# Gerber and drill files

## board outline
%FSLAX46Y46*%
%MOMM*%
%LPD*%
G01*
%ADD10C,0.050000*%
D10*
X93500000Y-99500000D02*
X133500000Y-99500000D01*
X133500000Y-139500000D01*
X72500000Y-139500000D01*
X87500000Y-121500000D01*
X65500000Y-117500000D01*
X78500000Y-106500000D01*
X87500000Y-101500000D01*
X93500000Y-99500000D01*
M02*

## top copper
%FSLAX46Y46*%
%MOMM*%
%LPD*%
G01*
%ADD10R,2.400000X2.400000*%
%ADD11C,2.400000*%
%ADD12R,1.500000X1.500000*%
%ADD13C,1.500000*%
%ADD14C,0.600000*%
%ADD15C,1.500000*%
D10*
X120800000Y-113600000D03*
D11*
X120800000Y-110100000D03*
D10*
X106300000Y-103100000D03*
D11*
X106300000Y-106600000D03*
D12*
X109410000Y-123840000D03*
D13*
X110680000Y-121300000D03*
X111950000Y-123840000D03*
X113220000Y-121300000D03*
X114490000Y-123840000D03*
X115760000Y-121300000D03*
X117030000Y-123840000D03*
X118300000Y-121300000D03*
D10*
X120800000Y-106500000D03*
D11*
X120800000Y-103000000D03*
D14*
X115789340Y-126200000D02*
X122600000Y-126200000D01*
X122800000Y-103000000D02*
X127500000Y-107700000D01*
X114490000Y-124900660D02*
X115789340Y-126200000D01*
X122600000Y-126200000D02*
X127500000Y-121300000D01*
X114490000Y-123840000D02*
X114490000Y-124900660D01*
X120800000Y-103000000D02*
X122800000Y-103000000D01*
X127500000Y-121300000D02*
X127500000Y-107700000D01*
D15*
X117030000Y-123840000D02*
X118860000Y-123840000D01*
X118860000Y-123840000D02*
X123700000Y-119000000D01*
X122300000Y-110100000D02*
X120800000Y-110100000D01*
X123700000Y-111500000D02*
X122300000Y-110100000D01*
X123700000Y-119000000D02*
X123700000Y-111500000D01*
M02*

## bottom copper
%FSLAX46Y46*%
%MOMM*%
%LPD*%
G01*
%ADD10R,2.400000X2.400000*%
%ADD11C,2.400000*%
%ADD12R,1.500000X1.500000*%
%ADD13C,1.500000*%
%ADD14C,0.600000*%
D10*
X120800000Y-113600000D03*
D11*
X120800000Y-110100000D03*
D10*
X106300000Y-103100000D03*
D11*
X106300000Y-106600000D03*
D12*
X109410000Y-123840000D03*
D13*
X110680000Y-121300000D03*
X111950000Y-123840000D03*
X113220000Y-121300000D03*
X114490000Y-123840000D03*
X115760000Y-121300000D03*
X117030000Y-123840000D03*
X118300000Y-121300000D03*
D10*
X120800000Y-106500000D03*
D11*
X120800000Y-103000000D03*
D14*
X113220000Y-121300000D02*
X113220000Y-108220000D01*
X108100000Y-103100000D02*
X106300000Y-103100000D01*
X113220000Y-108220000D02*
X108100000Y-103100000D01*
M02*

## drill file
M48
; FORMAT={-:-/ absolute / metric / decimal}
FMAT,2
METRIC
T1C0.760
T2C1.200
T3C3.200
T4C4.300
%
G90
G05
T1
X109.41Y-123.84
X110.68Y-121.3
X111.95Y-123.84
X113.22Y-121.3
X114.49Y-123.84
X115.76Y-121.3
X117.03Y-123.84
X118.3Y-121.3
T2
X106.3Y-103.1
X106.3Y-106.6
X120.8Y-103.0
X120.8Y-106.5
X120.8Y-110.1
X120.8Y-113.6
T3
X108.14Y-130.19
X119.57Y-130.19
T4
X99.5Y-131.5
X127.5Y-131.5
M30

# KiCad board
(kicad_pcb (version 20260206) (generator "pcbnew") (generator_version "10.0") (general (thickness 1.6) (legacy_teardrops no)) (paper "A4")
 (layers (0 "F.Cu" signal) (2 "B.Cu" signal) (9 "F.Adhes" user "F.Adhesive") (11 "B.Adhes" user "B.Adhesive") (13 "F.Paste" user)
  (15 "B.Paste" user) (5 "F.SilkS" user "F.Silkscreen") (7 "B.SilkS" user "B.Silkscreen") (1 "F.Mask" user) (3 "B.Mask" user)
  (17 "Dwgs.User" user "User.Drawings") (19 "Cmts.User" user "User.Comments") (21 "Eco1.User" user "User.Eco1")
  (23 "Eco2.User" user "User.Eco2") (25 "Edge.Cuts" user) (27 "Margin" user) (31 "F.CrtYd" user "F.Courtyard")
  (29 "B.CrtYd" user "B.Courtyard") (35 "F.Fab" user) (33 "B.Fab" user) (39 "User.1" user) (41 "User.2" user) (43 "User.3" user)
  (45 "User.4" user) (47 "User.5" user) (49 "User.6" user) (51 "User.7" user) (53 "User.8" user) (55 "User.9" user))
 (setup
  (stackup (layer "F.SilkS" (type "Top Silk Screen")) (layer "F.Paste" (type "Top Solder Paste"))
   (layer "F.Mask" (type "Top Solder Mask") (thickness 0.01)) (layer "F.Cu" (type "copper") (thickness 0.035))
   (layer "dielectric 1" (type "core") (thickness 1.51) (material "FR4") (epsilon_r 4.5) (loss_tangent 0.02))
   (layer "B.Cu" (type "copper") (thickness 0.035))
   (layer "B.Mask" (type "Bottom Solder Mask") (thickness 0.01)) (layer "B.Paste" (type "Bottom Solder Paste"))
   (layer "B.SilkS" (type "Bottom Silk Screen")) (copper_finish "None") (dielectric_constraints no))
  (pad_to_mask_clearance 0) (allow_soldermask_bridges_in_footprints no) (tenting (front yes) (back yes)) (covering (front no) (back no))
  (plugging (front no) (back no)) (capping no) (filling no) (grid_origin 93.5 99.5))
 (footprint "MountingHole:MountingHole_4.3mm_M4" (layer "F.Cu") (at 127.5 131.5)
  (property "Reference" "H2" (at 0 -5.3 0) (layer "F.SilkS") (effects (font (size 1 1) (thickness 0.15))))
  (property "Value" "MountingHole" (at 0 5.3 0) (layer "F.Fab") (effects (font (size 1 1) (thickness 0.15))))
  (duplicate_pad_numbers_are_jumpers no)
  (pad "" np_thru_hole circle (at 0 0) (size 4.3 4.3) (drill 4.3) (layers "*.Cu" "*.Mask")))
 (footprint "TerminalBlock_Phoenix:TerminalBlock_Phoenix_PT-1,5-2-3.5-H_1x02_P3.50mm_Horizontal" (layer "F.Cu") (at 120.8 113.6 90)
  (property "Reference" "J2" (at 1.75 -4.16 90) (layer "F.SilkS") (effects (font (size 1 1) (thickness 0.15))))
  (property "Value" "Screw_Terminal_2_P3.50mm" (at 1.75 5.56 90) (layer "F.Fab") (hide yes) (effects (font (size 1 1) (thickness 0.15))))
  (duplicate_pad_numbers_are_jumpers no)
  (pad "1" thru_hole rect (at 0 0 90) (size 2.4 2.4) (drill 1.2) (layers "*.Cu" "*.Mask") (remove_unused_layers no) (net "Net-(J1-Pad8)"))
  (pad "2" thru_hole circle (at 3.5 0 90) (size 2.4 2.4) (drill 1.2) (layers "*.Cu" "*.Mask") (remove_unused_layers no)
   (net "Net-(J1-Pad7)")))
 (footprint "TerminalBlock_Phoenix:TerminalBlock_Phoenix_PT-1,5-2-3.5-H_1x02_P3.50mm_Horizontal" (layer "F.Cu") (at 106.3 103.1 -90)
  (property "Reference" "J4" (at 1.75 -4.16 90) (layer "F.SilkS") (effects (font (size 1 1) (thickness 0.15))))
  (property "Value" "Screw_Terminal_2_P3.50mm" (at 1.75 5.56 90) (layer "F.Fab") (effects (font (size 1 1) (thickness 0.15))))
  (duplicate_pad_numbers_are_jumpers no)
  (pad "1" thru_hole rect (at 0 0 270) (size 2.4 2.4) (drill 1.2) (layers "*.Cu" "*.Mask") (remove_unused_layers no) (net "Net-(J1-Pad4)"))
  (pad "2" thru_hole circle (at 3.5 0 270) (size 2.4 2.4) (drill 1.2) (layers "*.Cu" "*.Mask") (remove_unused_layers no)
   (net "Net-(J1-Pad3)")))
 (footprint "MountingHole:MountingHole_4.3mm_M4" (layer "F.Cu") (at 99.5 131.5)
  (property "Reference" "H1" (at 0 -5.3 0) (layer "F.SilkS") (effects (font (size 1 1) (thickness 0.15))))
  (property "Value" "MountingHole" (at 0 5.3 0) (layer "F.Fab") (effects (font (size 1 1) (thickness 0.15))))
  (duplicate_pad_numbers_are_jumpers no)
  (pad "" np_thru_hole circle (at 0 0) (size 4.3 4.3) (drill 4.3) (layers "*.Cu" "*.Mask")))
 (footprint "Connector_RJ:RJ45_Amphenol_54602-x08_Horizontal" (layer "F.Cu") (at 109.41 123.84)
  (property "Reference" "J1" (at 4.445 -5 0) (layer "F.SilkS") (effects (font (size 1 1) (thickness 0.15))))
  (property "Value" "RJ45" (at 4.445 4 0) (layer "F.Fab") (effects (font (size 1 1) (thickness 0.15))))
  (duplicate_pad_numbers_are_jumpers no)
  (pad "" np_thru_hole circle (at -1.27 6.35) (size 3.2 3.2) (drill 3.2) (layers "*.Cu" "*.Mask"))
  (pad "" np_thru_hole circle (at 10.16 6.35) (size 3.2 3.2) (drill 3.2) (layers "*.Cu" "*.Mask"))
  (pad "1" thru_hole rect (at 0 0) (size 1.5 1.5) (drill 0.76) (layers "*.Cu" "*.Mask") (remove_unused_layers no)
   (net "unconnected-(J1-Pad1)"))
  (pad "2" thru_hole circle (at 1.27 -2.54) (size 1.5 1.5) (drill 0.76) (layers "*.Cu" "*.Mask") (remove_unused_layers no)
   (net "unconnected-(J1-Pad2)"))
  (pad "3" thru_hole circle (at 2.54 0) (size 1.5 1.5) (drill 0.76) (layers "*.Cu" "*.Mask") (remove_unused_layers no) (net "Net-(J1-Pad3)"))
  (pad "4" thru_hole circle (at 3.81 -2.54) (size 1.5 1.5) (drill 0.76) (layers "*.Cu" "*.Mask") (remove_unused_layers no)
   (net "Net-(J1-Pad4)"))
  (pad "5" thru_hole circle (at 5.08 0) (size 1.5 1.5) (drill 0.76) (layers "*.Cu" "*.Mask") (remove_unused_layers no) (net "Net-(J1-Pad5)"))
  (pad "6" thru_hole circle (at 6.35 -2.54) (size 1.5 1.5) (drill 0.76) (layers "*.Cu" "*.Mask") (remove_unused_layers no)
   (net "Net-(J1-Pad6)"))
  (pad "7" thru_hole circle (at 7.62 0) (size 1.5 1.5) (drill 0.76) (layers "*.Cu" "*.Mask") (remove_unused_layers no) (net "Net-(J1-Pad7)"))
  (pad "8" thru_hole circle (at 8.89 -2.54) (size 1.5 1.5) (drill 0.76) (layers "*.Cu" "*.Mask") (remove_unused_layers no)
   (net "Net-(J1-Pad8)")))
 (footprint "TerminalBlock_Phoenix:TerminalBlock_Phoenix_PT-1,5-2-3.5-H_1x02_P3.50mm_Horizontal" (layer "F.Cu") (at 120.8 106.5 90)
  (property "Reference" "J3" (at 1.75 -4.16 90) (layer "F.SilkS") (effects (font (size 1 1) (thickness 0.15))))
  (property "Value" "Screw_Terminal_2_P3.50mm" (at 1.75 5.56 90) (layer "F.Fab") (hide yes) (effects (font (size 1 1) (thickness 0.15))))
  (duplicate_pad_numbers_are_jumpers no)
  (pad "1" thru_hole rect (at 0 0 90) (size 2.4 2.4) (drill 1.2) (layers "*.Cu" "*.Mask") (remove_unused_layers no) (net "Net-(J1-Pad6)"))
  (pad "2" thru_hole circle (at 3.5 0 90) (size 2.4 2.4) (drill 1.2) (layers "*.Cu" "*.Mask") (remove_unused_layers no)
   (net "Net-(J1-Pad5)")))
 (gr_poly
  (pts (xy 93.5 99.5) (xy 133.5 99.5) (xy 133.5 139.5) (xy 72.5 139.5) (xy 87.5 121.5) (xy 65.5 117.5) (xy 78.5 106.5) (xy 87.5 101.5))
  (stroke (width 0.05) (type solid)) (fill no) (layer "Edge.Cuts"))
 (segment (start 113.22 121.3) (end 113.22 108.22) (width 0.6) (layer "B.Cu") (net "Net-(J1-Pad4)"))
 (segment (start 108.1 103.1) (end 106.3 103.1) (width 0.6) (layer "B.Cu") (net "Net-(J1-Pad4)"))
 (segment (start 113.22 108.22) (end 108.1 103.1) (width 0.6) (layer "B.Cu") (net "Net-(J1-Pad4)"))
 (segment (start 115.78934 126.2) (end 122.6 126.2) (width 0.6) (layer "F.Cu") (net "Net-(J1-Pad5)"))
 (segment (start 122.8 103) (end 127.5 107.7) (width 0.6) (layer "F.Cu") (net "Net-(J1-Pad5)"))
 (segment (start 114.49 124.90066) (end 115.78934 126.2) (width 0.6) (layer "F.Cu") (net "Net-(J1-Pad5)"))
 (segment (start 122.6 126.2) (end 127.5 121.3) (width 0.6) (layer "F.Cu") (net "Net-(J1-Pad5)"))
 (segment (start 114.49 123.84) (end 114.49 124.90066) (width 0.6) (layer "F.Cu") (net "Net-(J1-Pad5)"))
 (segment (start 120.8 103) (end 122.8 103) (width 0.6) (layer "F.Cu") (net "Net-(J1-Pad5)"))
 (segment (start 127.5 121.3) (end 127.5 107.7) (width 0.6) (layer "F.Cu") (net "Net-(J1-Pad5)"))
 (segment (start 117.03 123.84) (end 118.86 123.84) (width 1.5) (layer "F.Cu") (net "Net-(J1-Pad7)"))
 (segment (start 118.86 123.84) (end 123.7 119) (width 1.5) (layer "F.Cu") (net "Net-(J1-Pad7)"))
 (segment (start 122.3 110.1) (end 120.8 110.1) (width 1.5) (layer "F.Cu") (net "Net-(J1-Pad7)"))
 (segment (start 123.7 111.5) (end 122.3 110.1) (width 1.5) (layer "F.Cu") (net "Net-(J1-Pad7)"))
 (segment (start 123.7 119) (end 123.7 111.5) (width 1.5) (layer "F.Cu") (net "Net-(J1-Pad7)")))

